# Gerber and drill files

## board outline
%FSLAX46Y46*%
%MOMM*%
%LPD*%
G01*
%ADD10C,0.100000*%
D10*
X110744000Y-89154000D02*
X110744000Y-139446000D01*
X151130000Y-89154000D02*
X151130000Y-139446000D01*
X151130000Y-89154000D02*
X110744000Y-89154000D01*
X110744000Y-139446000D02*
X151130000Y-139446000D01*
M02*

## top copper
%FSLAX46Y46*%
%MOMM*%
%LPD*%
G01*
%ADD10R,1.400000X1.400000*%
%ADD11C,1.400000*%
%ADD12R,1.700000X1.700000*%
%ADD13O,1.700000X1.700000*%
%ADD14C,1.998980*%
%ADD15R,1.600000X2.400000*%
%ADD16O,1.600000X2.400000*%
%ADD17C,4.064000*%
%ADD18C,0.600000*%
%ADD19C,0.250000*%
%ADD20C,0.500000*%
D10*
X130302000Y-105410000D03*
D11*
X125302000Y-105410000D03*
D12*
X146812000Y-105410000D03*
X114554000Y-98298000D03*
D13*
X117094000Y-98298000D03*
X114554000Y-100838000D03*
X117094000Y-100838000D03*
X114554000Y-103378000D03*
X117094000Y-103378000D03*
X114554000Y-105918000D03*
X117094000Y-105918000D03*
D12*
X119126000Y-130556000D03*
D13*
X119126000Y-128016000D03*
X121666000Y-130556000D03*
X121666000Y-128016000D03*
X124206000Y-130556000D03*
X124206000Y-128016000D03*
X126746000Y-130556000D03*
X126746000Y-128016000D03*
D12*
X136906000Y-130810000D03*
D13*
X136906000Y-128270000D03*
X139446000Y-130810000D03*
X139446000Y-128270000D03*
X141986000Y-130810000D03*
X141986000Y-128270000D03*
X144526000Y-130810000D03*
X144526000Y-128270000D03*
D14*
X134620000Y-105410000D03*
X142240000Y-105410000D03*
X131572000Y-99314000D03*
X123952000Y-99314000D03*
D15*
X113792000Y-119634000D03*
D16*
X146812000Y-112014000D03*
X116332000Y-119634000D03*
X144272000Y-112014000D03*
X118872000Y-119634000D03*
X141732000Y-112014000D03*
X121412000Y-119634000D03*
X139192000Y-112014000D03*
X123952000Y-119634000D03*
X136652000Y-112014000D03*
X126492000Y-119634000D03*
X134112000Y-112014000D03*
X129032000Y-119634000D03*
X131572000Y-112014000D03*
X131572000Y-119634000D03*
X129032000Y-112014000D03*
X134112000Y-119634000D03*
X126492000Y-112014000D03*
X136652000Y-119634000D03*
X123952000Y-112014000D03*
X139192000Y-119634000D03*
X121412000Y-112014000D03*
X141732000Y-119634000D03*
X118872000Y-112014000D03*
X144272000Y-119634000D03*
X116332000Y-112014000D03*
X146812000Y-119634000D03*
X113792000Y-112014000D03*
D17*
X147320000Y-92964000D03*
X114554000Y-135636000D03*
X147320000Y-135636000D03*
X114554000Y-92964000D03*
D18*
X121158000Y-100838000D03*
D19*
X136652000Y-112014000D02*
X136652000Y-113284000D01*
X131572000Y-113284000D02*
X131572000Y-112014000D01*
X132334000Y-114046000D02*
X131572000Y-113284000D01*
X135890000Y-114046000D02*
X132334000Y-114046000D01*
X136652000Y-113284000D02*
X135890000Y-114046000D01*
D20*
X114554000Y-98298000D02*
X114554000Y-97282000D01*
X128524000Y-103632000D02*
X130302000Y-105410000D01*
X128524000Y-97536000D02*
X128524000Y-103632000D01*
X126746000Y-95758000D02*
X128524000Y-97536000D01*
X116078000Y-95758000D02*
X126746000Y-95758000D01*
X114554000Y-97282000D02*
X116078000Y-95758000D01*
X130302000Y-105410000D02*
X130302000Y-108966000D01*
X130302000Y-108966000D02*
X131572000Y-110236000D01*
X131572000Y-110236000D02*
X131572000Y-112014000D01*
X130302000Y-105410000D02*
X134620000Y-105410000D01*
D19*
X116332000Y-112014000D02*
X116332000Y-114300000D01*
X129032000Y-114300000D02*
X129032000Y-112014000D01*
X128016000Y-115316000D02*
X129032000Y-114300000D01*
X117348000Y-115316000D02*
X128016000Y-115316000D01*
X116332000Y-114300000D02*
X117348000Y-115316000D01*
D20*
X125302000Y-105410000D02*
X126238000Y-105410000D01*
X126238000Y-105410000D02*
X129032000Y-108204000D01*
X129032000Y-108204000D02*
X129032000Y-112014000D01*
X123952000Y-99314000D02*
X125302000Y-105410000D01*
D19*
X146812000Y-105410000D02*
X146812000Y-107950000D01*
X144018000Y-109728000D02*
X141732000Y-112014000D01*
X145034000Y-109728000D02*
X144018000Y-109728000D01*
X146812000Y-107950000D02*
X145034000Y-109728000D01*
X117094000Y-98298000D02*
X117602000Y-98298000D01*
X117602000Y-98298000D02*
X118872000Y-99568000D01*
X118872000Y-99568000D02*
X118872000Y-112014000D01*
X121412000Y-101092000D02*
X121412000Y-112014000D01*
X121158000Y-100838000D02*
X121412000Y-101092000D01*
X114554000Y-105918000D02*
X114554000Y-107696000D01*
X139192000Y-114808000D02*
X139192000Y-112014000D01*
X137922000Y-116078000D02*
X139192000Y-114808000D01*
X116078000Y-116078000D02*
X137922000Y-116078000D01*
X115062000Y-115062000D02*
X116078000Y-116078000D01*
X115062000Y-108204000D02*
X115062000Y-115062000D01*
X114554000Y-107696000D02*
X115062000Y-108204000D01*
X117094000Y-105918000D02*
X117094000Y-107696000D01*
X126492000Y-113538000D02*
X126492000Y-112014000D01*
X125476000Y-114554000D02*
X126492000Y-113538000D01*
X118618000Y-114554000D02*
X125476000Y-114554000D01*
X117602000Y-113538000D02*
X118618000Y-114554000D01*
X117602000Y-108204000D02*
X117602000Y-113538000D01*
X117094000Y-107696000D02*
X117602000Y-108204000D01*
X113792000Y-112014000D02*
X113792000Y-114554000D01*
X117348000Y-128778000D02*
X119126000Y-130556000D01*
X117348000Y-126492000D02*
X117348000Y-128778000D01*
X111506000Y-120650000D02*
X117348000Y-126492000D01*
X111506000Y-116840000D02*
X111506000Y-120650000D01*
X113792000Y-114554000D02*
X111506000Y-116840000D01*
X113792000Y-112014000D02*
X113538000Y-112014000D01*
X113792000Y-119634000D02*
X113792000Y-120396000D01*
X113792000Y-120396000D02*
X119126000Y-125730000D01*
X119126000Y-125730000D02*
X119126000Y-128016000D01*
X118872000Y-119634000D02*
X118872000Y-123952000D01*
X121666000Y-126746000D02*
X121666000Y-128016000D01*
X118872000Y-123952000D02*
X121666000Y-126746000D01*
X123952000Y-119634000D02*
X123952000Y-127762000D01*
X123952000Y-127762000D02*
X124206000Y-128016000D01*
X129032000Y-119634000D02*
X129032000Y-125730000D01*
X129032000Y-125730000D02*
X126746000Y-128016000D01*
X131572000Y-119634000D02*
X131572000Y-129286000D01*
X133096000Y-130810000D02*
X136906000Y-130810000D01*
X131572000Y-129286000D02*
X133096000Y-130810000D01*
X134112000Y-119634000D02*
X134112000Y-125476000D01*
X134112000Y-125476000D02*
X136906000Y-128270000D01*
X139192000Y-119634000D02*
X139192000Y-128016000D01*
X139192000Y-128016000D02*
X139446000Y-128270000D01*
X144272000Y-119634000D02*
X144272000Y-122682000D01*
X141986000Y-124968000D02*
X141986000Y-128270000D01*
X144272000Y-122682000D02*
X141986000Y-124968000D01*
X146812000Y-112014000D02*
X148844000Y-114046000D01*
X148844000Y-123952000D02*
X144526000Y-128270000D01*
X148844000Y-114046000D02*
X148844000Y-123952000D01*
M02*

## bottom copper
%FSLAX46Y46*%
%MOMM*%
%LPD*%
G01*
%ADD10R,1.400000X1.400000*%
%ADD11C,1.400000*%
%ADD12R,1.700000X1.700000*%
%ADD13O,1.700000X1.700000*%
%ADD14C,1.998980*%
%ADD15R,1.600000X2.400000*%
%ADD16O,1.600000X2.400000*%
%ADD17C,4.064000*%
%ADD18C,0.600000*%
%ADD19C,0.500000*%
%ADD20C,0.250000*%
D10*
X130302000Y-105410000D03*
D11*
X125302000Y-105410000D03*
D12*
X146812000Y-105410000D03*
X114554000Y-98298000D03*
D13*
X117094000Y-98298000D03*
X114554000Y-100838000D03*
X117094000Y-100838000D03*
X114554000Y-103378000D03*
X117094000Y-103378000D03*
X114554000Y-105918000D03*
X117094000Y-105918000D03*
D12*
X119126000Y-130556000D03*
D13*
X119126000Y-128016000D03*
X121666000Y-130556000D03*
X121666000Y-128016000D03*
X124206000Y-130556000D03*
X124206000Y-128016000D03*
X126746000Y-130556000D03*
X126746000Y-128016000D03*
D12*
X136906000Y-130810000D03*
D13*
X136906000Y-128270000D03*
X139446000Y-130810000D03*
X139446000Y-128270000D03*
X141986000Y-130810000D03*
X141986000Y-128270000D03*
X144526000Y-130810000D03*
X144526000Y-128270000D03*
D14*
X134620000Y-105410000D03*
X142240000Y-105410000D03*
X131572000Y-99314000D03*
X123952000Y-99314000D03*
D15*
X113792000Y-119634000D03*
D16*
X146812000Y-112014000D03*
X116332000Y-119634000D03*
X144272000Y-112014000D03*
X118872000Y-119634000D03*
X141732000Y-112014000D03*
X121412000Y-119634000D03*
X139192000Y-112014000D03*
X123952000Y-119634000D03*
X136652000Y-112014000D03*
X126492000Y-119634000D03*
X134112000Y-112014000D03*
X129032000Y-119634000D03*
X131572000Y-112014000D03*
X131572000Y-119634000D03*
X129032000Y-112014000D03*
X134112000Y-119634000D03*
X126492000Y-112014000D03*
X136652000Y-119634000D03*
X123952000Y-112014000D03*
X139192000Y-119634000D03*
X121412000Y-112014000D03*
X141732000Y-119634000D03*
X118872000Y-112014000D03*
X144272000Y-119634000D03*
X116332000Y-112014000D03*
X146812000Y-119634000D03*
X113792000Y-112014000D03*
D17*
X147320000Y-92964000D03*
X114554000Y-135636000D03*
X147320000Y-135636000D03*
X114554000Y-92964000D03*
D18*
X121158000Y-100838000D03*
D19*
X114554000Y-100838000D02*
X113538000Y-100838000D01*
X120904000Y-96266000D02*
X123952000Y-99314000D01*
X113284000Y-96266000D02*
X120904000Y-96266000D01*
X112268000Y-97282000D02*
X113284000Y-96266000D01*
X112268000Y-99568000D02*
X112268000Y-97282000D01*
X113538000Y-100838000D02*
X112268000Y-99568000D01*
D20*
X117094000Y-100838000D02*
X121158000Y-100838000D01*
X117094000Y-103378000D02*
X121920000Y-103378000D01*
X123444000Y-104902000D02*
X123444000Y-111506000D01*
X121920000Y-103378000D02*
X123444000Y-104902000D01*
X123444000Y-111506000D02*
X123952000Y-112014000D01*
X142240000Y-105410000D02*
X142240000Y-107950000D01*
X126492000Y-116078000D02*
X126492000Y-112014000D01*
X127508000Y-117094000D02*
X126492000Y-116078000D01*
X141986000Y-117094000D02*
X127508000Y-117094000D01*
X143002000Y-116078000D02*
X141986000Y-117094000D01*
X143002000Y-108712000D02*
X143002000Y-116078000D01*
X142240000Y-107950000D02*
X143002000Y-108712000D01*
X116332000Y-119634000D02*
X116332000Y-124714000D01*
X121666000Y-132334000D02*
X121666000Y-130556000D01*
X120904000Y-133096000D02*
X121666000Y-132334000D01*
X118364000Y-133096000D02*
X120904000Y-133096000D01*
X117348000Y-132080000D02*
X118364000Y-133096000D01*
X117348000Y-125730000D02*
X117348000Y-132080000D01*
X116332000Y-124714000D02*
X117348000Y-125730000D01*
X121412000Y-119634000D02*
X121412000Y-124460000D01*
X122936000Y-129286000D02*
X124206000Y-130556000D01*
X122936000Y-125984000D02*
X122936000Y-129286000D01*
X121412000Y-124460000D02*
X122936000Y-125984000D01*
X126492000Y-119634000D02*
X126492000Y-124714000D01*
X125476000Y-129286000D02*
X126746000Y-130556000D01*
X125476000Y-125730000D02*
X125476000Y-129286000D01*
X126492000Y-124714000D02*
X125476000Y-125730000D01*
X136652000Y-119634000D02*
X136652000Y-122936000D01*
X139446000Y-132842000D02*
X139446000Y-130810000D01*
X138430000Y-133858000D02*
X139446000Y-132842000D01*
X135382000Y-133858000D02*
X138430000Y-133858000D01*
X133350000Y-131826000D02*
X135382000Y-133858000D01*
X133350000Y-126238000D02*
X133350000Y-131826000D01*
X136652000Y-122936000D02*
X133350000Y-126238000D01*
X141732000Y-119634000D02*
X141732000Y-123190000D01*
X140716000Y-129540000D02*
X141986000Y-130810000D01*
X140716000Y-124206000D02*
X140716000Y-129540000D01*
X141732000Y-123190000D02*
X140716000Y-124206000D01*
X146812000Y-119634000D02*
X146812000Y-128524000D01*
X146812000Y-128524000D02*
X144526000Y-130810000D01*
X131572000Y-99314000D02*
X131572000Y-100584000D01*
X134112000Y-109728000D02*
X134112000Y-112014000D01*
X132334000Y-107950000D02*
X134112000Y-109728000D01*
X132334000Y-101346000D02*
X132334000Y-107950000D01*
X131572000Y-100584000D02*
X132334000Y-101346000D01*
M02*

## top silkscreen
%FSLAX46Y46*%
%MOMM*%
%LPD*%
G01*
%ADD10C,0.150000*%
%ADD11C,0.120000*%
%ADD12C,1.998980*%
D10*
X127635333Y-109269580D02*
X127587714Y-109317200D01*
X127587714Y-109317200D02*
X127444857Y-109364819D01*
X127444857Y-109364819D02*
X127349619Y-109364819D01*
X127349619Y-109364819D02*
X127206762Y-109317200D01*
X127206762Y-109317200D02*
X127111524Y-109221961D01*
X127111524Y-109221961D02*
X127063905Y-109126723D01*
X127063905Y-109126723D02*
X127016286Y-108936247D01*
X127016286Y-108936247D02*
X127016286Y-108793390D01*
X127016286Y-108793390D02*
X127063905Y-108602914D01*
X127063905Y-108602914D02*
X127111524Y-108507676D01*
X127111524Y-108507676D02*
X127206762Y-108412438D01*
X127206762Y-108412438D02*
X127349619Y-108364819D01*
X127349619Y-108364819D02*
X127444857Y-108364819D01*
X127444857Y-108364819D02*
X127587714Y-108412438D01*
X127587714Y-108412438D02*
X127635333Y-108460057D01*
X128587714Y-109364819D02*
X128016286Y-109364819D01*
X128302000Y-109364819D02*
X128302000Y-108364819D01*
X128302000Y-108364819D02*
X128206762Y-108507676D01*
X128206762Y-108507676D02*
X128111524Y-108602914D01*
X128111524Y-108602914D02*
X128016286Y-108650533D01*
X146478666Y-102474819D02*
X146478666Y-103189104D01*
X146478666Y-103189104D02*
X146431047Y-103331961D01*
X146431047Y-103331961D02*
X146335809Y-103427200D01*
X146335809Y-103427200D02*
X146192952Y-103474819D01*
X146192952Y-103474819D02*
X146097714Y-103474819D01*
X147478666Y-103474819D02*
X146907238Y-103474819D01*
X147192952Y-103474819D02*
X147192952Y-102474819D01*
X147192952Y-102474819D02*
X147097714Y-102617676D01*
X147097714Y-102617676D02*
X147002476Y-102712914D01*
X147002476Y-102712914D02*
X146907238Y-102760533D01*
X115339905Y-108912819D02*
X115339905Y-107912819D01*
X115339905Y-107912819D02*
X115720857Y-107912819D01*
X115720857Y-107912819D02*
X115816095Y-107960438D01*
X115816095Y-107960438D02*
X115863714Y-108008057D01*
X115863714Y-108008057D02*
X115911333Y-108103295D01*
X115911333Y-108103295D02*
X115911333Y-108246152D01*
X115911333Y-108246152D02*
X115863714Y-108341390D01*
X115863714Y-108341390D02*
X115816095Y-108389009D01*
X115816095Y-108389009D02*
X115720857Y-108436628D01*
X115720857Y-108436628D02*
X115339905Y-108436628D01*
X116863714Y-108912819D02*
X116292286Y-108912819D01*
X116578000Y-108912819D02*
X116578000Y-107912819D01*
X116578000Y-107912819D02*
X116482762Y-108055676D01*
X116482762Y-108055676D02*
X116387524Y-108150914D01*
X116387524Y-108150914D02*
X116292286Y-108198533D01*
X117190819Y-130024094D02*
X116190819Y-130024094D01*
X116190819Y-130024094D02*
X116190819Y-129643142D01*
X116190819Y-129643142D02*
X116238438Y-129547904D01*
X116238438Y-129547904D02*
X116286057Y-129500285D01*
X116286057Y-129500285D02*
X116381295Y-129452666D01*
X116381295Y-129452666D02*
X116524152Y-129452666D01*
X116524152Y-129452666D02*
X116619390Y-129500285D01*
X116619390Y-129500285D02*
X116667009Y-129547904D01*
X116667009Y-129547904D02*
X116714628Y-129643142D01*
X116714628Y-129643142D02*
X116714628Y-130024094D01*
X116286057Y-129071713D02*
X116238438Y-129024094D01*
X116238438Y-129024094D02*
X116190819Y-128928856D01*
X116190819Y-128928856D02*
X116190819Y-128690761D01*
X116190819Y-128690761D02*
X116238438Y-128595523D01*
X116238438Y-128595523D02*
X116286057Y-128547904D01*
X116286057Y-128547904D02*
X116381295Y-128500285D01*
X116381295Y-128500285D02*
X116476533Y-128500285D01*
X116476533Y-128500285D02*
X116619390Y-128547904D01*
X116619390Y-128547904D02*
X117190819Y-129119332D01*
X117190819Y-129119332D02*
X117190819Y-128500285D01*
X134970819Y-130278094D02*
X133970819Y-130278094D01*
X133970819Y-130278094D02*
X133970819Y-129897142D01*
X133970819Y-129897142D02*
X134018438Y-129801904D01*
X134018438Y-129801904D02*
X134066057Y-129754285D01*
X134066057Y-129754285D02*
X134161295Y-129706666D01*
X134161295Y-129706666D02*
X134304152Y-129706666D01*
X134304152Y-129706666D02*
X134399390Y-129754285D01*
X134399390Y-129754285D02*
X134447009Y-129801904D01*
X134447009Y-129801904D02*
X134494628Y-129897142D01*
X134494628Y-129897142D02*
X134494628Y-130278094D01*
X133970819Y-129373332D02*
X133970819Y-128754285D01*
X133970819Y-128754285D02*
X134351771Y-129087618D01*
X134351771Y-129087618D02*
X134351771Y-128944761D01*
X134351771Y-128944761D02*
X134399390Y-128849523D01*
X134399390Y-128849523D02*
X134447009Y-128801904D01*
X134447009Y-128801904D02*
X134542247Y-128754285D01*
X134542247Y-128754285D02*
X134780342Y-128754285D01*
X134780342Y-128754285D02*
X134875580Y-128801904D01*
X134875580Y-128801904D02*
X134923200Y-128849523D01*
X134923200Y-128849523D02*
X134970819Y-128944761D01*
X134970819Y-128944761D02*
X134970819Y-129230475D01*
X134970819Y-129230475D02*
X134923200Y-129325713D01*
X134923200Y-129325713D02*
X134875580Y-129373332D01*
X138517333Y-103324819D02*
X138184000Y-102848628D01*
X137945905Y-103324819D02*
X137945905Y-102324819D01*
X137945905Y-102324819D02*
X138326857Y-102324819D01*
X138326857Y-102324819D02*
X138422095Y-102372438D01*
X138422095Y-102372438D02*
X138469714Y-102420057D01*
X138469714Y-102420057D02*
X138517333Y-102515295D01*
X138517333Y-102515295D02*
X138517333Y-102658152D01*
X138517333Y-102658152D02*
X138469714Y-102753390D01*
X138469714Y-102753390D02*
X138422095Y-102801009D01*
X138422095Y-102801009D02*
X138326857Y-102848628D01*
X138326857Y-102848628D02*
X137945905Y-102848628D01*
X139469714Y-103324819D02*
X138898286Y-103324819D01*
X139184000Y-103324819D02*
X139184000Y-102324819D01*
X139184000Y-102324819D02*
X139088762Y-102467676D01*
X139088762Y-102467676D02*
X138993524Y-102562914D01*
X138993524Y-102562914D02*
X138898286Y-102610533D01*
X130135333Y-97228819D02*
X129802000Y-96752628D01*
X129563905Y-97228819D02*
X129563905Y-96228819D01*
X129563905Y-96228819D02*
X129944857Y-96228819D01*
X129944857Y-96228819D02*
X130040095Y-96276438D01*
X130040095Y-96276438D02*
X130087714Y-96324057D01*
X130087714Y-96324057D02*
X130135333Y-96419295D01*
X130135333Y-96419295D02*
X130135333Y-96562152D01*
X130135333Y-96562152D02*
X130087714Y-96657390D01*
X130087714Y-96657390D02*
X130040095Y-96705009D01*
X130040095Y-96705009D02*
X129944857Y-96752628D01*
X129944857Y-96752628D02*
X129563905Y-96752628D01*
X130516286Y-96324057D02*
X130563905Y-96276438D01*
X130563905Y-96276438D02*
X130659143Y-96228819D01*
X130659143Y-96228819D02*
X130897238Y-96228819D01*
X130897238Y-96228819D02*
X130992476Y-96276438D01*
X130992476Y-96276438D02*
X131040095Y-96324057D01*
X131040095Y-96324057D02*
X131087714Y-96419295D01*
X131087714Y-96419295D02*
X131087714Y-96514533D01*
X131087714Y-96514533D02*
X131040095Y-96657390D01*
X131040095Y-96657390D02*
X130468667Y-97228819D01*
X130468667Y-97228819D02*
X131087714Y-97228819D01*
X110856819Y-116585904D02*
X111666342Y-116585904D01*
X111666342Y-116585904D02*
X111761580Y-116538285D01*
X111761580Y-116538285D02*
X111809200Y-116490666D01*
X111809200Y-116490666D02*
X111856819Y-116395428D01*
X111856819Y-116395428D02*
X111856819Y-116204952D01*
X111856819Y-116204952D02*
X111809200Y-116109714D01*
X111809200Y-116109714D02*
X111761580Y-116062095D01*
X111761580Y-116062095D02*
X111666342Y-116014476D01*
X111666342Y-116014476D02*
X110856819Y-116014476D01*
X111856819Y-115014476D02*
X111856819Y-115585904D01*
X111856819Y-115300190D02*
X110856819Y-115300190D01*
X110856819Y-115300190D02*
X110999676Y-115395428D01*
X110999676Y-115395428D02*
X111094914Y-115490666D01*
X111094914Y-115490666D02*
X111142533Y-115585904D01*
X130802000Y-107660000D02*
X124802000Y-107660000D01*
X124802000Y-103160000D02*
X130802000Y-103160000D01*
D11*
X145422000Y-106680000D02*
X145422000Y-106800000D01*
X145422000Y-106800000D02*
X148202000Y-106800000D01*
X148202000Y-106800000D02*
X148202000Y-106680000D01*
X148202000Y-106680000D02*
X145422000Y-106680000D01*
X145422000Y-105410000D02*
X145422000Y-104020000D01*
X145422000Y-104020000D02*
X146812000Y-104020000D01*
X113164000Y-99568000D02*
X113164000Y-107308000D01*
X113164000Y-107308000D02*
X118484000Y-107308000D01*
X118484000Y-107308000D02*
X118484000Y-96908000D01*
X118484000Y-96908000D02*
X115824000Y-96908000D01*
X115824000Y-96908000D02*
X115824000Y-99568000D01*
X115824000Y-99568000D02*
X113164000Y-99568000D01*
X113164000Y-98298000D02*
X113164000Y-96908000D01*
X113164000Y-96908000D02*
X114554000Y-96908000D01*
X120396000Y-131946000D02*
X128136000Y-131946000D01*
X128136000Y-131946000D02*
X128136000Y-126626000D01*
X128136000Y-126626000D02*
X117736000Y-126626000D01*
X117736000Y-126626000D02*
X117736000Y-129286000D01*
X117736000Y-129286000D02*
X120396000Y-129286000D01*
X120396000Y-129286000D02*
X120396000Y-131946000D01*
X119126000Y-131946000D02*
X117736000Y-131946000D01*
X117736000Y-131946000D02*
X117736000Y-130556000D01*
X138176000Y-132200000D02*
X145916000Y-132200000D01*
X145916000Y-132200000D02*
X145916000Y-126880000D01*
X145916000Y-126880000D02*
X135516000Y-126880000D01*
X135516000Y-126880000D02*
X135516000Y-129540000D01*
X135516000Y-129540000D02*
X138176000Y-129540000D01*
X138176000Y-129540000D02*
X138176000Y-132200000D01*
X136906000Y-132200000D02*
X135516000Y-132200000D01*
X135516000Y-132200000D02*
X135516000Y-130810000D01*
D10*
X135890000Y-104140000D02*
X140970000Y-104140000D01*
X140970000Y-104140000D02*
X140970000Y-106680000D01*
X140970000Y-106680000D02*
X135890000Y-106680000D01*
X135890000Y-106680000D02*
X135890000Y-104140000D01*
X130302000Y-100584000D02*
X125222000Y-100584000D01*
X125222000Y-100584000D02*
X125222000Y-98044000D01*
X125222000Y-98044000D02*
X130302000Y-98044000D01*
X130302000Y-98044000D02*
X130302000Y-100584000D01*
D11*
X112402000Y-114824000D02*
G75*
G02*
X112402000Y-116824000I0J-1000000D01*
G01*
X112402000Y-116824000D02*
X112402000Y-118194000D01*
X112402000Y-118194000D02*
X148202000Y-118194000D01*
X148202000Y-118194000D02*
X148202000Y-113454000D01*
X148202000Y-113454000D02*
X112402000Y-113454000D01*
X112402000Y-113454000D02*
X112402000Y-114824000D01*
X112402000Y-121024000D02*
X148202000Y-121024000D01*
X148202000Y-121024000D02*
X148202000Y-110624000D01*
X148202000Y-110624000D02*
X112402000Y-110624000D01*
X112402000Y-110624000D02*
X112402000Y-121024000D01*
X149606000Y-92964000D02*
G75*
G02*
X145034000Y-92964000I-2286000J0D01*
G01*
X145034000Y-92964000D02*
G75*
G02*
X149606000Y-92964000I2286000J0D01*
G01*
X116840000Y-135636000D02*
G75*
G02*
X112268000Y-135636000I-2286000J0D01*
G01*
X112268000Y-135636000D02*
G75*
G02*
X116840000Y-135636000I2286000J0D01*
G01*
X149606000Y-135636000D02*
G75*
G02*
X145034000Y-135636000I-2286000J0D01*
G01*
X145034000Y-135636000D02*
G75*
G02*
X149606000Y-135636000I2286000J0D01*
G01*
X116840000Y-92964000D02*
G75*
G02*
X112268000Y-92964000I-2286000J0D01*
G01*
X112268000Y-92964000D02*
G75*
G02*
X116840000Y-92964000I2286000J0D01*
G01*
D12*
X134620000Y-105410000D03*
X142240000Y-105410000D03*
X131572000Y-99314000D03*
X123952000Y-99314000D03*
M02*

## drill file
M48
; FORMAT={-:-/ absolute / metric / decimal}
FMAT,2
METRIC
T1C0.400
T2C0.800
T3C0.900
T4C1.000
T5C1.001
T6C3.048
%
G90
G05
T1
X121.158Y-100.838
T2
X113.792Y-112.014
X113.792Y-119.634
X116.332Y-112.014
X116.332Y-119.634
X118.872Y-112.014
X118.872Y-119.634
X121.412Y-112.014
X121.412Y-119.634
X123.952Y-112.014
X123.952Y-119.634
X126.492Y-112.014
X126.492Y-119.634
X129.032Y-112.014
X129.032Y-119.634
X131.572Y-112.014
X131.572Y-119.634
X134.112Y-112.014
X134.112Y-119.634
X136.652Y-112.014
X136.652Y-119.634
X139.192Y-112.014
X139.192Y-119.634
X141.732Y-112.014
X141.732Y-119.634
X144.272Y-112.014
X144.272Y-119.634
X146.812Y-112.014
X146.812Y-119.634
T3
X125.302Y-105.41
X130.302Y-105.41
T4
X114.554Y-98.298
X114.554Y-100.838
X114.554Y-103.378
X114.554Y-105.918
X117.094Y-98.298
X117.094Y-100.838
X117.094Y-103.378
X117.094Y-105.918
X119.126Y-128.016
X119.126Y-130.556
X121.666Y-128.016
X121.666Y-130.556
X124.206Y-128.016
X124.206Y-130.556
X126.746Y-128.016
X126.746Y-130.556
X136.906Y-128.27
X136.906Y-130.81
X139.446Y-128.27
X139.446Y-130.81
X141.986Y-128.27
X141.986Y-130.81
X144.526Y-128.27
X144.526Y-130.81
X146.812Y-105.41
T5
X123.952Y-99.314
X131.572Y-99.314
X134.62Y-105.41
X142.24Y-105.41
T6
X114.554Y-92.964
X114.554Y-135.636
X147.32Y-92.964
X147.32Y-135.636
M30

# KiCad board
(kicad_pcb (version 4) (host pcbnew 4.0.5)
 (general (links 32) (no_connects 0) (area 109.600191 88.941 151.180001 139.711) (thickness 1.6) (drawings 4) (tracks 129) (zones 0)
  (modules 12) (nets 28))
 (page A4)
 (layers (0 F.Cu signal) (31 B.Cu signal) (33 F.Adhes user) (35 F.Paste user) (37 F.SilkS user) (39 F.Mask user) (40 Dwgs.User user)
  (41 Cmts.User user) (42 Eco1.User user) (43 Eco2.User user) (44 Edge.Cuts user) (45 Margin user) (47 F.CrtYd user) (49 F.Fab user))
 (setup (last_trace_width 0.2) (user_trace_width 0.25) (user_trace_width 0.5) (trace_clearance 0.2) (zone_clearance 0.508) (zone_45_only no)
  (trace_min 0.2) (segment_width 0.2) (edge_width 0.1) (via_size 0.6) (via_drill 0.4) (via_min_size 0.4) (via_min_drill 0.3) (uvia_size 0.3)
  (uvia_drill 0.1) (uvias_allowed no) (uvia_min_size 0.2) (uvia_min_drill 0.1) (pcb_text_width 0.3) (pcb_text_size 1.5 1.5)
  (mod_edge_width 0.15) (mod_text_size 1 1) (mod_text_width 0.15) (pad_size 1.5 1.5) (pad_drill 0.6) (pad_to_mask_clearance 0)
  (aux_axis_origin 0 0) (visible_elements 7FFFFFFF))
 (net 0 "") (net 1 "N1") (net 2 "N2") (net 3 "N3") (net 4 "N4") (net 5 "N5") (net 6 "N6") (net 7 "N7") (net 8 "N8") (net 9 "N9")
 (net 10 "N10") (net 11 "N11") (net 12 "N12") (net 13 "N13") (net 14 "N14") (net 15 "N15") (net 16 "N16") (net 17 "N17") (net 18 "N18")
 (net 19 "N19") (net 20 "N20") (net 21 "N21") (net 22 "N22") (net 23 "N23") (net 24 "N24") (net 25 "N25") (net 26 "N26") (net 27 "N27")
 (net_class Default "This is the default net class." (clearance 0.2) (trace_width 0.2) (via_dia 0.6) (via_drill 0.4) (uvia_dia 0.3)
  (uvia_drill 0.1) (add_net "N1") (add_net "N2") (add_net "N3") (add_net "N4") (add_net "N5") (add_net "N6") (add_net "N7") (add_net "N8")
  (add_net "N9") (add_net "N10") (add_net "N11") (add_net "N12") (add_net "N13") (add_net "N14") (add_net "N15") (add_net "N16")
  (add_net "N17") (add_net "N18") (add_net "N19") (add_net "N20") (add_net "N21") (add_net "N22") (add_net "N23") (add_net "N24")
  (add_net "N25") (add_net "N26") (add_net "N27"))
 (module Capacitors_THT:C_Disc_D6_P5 (layer F.Cu) (at 130.302 105.41 180)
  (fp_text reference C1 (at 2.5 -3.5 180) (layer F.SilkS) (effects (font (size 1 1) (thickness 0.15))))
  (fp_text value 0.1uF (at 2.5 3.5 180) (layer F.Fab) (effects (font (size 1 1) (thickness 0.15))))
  (fp_line (start -0.5 -2.25) (end 5.5 -2.25) (layer F.SilkS) (width 0.15))
  (fp_line (start 5.5 2.25) (end -0.5 2.25) (layer F.SilkS) (width 0.15))
  (pad 1 thru_hole rect (at 0 0 180) (size 1.4 1.4) (drill 0.9) (layers *.Cu *.Mask) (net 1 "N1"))
  (pad 2 thru_hole circle (at 5 0 180) (size 1.4 1.4) (drill 0.9) (layers *.Cu *.Mask) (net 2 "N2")))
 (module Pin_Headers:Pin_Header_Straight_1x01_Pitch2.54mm (layer F.Cu) (at 146.812 105.41)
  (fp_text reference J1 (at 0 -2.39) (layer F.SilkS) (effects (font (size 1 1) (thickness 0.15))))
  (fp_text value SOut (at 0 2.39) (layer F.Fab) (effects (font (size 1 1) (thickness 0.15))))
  (fp_line (start -1.39 1.27) (end -1.39 1.39) (layer F.SilkS) (width 0.12))
  (fp_line (start -1.39 1.39) (end 1.39 1.39) (layer F.SilkS) (width 0.12))
  (fp_line (start 1.39 1.39) (end 1.39 1.27) (layer F.SilkS) (width 0.12))
  (fp_line (start 1.39 1.27) (end -1.39 1.27) (layer F.SilkS) (width 0.12))
  (fp_line (start -1.39 0) (end -1.39 -1.39) (layer F.SilkS) (width 0.12))
  (fp_line (start -1.39 -1.39) (end 0 -1.39) (layer F.SilkS) (width 0.12))
  (pad 1 thru_hole rect (at 0 0) (size 1.7 1.7) (drill 1) (layers *.Cu *.Mask) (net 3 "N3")))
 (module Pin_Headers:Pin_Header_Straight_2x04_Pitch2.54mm (layer F.Cu) (at 114.554 98.298)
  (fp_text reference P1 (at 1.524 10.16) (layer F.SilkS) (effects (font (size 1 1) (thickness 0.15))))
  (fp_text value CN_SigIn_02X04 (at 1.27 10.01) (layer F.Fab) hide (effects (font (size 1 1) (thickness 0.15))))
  (fp_line (start -1.39 1.27) (end -1.39 9.01) (layer F.SilkS) (width 0.12))
  (fp_line (start -1.39 9.01) (end 3.93 9.01) (layer F.SilkS) (width 0.12))
  (fp_line (start 3.93 9.01) (end 3.93 -1.39) (layer F.SilkS) (width 0.12))
  (fp_line (start 3.93 -1.39) (end 1.27 -1.39) (layer F.SilkS) (width 0.12))
  (fp_line (start 1.27 -1.39) (end 1.27 1.27) (layer F.SilkS) (width 0.12))
  (fp_line (start 1.27 1.27) (end -1.39 1.27) (layer F.SilkS) (width 0.12))
  (fp_line (start -1.39 0) (end -1.39 -1.39) (layer F.SilkS) (width 0.12))
  (fp_line (start -1.39 -1.39) (end 0 -1.39) (layer F.SilkS) (width 0.12))
  (pad 1 thru_hole rect (at 0 0) (size 1.7 1.7) (drill 1) (layers *.Cu *.Mask) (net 1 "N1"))
  (pad 2 thru_hole oval (at 2.54 0) (size 1.7 1.7) (drill 1) (layers *.Cu *.Mask) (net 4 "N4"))
  (pad 3 thru_hole oval (at 0 2.54) (size 1.7 1.7) (drill 1) (layers *.Cu *.Mask) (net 2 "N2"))
  (pad 4 thru_hole oval (at 2.54 2.54) (size 1.7 1.7) (drill 1) (layers *.Cu *.Mask) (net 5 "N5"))
  (pad 5 thru_hole oval (at 0 5.08) (size 1.7 1.7) (drill 1) (layers *.Cu *.Mask) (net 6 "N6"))
  (pad 6 thru_hole oval (at 2.54 5.08) (size 1.7 1.7) (drill 1) (layers *.Cu *.Mask) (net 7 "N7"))
  (pad 7 thru_hole oval (at 0 7.62) (size 1.7 1.7) (drill 1) (layers *.Cu *.Mask) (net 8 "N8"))
  (pad 8 thru_hole oval (at 2.54 7.62) (size 1.7 1.7) (drill 1) (layers *.Cu *.Mask) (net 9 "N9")))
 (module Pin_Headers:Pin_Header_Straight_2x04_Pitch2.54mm (layer F.Cu) (at 119.126 130.556 90)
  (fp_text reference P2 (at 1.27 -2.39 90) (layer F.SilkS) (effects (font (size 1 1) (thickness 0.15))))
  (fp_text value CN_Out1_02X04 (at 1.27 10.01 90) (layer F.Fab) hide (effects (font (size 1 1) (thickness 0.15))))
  (fp_line (start -1.39 1.27) (end -1.39 9.01) (layer F.SilkS) (width 0.12))
  (fp_line (start -1.39 9.01) (end 3.93 9.01) (layer F.SilkS) (width 0.12))
  (fp_line (start 3.93 9.01) (end 3.93 -1.39) (layer F.SilkS) (width 0.12))
  (fp_line (start 3.93 -1.39) (end 1.27 -1.39) (layer F.SilkS) (width 0.12))
  (fp_line (start 1.27 -1.39) (end 1.27 1.27) (layer F.SilkS) (width 0.12))
  (fp_line (start 1.27 1.27) (end -1.39 1.27) (layer F.SilkS) (width 0.12))
  (fp_line (start -1.39 0) (end -1.39 -1.39) (layer F.SilkS) (width 0.12))
  (fp_line (start -1.39 -1.39) (end 0 -1.39) (layer F.SilkS) (width 0.12))
  (pad 1 thru_hole rect (at 0 0 90) (size 1.7 1.7) (drill 1) (layers *.Cu *.Mask) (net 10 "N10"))
  (pad 2 thru_hole oval (at 2.54 0 90) (size 1.7 1.7) (drill 1) (layers *.Cu *.Mask) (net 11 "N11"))
  (pad 3 thru_hole oval (at 0 2.54 90) (size 1.7 1.7) (drill 1) (layers *.Cu *.Mask) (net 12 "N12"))
  (pad 4 thru_hole oval (at 2.54 2.54 90) (size 1.7 1.7) (drill 1) (layers *.Cu *.Mask) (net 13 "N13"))
  (pad 5 thru_hole oval (at 0 5.08 90) (size 1.7 1.7) (drill 1) (layers *.Cu *.Mask) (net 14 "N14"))
  (pad 6 thru_hole oval (at 2.54 5.08 90) (size 1.7 1.7) (drill 1) (layers *.Cu *.Mask) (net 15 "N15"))
  (pad 7 thru_hole oval (at 0 7.62 90) (size 1.7 1.7) (drill 1) (layers *.Cu *.Mask) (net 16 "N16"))
  (pad 8 thru_hole oval (at 2.54 7.62 90) (size 1.7 1.7) (drill 1) (layers *.Cu *.Mask) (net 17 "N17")))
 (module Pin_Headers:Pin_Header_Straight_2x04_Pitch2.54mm (layer F.Cu) (at 136.906 130.81 90)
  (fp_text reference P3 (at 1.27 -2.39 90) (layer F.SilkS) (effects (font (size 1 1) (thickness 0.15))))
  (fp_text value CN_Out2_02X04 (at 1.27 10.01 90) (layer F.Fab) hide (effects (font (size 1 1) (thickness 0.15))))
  (fp_line (start -1.39 1.27) (end -1.39 9.01) (layer F.SilkS) (width 0.12))
  (fp_line (start -1.39 9.01) (end 3.93 9.01) (layer F.SilkS) (width 0.12))
  (fp_line (start 3.93 9.01) (end 3.93 -1.39) (layer F.SilkS) (width 0.12))
  (fp_line (start 3.93 -1.39) (end 1.27 -1.39) (layer F.SilkS) (width 0.12))
  (fp_line (start 1.27 -1.39) (end 1.27 1.27) (layer F.SilkS) (width 0.12))
  (fp_line (start 1.27 1.27) (end -1.39 1.27) (layer F.SilkS) (width 0.12))
  (fp_line (start -1.39 0) (end -1.39 -1.39) (layer F.SilkS) (width 0.12))
  (fp_line (start -1.39 -1.39) (end 0 -1.39) (layer F.SilkS) (width 0.12))
  (pad 1 thru_hole rect (at 0 0 90) (size 1.7 1.7) (drill 1) (layers *.Cu *.Mask) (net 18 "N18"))
  (pad 2 thru_hole oval (at 2.54 0 90) (size 1.7 1.7) (drill 1) (layers *.Cu *.Mask) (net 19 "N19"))
  (pad 3 thru_hole oval (at 0 2.54 90) (size 1.7 1.7) (drill 1) (layers *.Cu *.Mask) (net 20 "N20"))
  (pad 4 thru_hole oval (at 2.54 2.54 90) (size 1.7 1.7) (drill 1) (layers *.Cu *.Mask) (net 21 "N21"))
  (pad 5 thru_hole oval (at 0 5.08 90) (size 1.7 1.7) (drill 1) (layers *.Cu *.Mask) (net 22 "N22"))
  (pad 6 thru_hole oval (at 2.54 5.08 90) (size 1.7 1.7) (drill 1) (layers *.Cu *.Mask) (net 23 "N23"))
  (pad 7 thru_hole oval (at 0 7.62 90) (size 1.7 1.7) (drill 1) (layers *.Cu *.Mask) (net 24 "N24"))
  (pad 8 thru_hole oval (at 2.54 7.62 90) (size 1.7 1.7) (drill 1) (layers *.Cu *.Mask) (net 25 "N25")))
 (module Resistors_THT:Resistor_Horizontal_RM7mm (layer F.Cu) (at 134.62 105.41)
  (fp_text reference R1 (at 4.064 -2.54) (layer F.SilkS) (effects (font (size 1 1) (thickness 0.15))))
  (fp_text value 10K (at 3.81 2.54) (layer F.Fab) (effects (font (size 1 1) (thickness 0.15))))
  (fp_line (start 1.27 -1.27) (end 6.35 -1.27) (layer F.SilkS) (width 0.15))
  (fp_line (start 6.35 -1.27) (end 6.35 1.27) (layer F.SilkS) (width 0.15))
  (fp_line (start 6.35 1.27) (end 1.27 1.27) (layer F.SilkS) (width 0.15))
  (fp_line (start 1.27 1.27) (end 1.27 -1.27) (layer F.SilkS) (width 0.15))
  (pad 1 thru_hole circle (at 0 0) (size 1.99898 1.99898) (drill 1.00076) (layers *.Cu *.SilkS *.Mask) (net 1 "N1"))
  (pad 2 thru_hole circle (at 7.62 0) (size 1.99898 1.99898) (drill 1.00076) (layers *.Cu *.SilkS *.Mask) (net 9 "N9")))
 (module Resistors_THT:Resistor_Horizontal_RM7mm (layer F.Cu) (at 131.572 99.314 180)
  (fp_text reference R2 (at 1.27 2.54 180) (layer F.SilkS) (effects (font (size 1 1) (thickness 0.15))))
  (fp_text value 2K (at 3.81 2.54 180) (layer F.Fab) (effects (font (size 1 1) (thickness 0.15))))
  (fp_line (start 1.27 -1.27) (end 6.35 -1.27) (layer F.SilkS) (width 0.15))
  (fp_line (start 6.35 -1.27) (end 6.35 1.27) (layer F.SilkS) (width 0.15))
  (fp_line (start 6.35 1.27) (end 1.27 1.27) (layer F.SilkS) (width 0.15))
  (fp_line (start 1.27 1.27) (end 1.27 -1.27) (layer F.SilkS) (width 0.15))
  (pad 1 thru_hole circle (at 0 0 180) (size 1.99898 1.99898) (drill 1.00076) (layers *.Cu *.SilkS *.Mask) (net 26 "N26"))
  (pad 2 thru_hole circle (at 7.62 0 180) (size 1.99898 1.99898) (drill 1.00076) (layers *.Cu *.SilkS *.Mask) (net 2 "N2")))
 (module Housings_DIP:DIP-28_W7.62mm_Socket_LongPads (layer F.Cu) (at 113.792 119.634 90)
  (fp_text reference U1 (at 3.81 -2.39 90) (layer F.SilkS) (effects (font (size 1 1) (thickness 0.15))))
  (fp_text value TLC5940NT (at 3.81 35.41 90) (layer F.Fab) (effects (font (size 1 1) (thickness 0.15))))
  (fp_arc (start 3.81 -1.39) (end 2.81 -1.39) (angle -180) (layer F.SilkS) (width 0.12))
  (fp_line (start 2.81 -1.39) (end 1.44 -1.39) (layer F.SilkS) (width 0.12))
  (fp_line (start 1.44 -1.39) (end 1.44 34.41) (layer F.SilkS) (width 0.12))
  (fp_line (start 1.44 34.41) (end 6.18 34.41) (layer F.SilkS) (width 0.12))
  (fp_line (start 6.18 34.41) (end 6.18 -1.39) (layer F.SilkS) (width 0.12))
  (fp_line (start 6.18 -1.39) (end 4.81 -1.39) (layer F.SilkS) (width 0.12))
  (fp_line (start -1.39 -1.39) (end -1.39 34.41) (layer F.SilkS) (width 0.12))
  (fp_line (start -1.39 34.41) (end 9.01 34.41) (layer F.SilkS) (width 0.12))
  (fp_line (start 9.01 34.41) (end 9.01 -1.39) (layer F.SilkS) (width 0.12))
  (fp_line (start 9.01 -1.39) (end -1.39 -1.39) (layer F.SilkS) (width 0.12))
  (pad 1 thru_hole rect (at 0 0 90) (size 2.4 1.6) (drill 0.8) (layers *.Cu *.Mask) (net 11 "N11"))
  (pad 15 thru_hole oval (at 7.62 33.02 90) (size 2.4 1.6) (drill 0.8) (layers *.Cu *.Mask) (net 25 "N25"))
  (pad 2 thru_hole oval (at 0 2.54 90) (size 2.4 1.6) (drill 0.8) (layers *.Cu *.Mask) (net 12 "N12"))
  (pad 16 thru_hole oval (at 7.62 30.48 90) (size 2.4 1.6) (drill 0.8) (layers *.Cu *.Mask) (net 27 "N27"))
  (pad 3 thru_hole oval (at 0 5.08 90) (size 2.4 1.6) (drill 0.8) (layers *.Cu *.Mask) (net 13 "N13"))
  (pad 17 thru_hole oval (at 7.62 27.94 90) (size 2.4 1.6) (drill 0.8) (layers *.Cu *.Mask) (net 3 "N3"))
  (pad 4 thru_hole oval (at 0 7.62 90) (size 2.4 1.6) (drill 0.8) (layers *.Cu *.Mask) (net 14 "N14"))
  (pad 18 thru_hole oval (at 7.62 25.4 90) (size 2.4 1.6) (drill 0.8) (layers *.Cu *.Mask) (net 8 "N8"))
  (pad 5 thru_hole oval (at 0 10.16 90) (size 2.4 1.6) (drill 0.8) (layers *.Cu *.Mask) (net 15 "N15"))
  (pad 19 thru_hole oval (at 7.62 22.86 90) (size 2.4 1.6) (drill 0.8) (layers *.Cu *.Mask) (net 1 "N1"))
  (pad 6 thru_hole oval (at 0 12.7 90) (size 2.4 1.6) (drill 0.8) (layers *.Cu *.Mask) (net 16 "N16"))
  (pad 20 thru_hole oval (at 7.62 20.32 90) (size 2.4 1.6) (drill 0.8) (layers *.Cu *.Mask) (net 26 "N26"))
  (pad 7 thru_hole oval (at 0 15.24 90) (size 2.4 1.6) (drill 0.8) (layers *.Cu *.Mask) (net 17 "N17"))
  (pad 21 thru_hole oval (at 7.62 17.78 90) (size 2.4 1.6) (drill 0.8) (layers *.Cu *.Mask) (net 1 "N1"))
  (pad 8 thru_hole oval (at 0 17.78 90) (size 2.4 1.6) (drill 0.8) (layers *.Cu *.Mask) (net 18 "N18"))
  (pad 22 thru_hole oval (at 7.62 15.24 90) (size 2.4 1.6) (drill 0.8) (layers *.Cu *.Mask) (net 2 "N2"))
  (pad 9 thru_hole oval (at 0 20.32 90) (size 2.4 1.6) (drill 0.8) (layers *.Cu *.Mask) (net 19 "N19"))
  (pad 23 thru_hole oval (at 7.62 12.7 90) (size 2.4 1.6) (drill 0.8) (layers *.Cu *.Mask) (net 9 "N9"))
  (pad 10 thru_hole oval (at 0 22.86 90) (size 2.4 1.6) (drill 0.8) (layers *.Cu *.Mask) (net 20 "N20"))
  (pad 24 thru_hole oval (at 7.62 10.16 90) (size 2.4 1.6) (drill 0.8) (layers *.Cu *.Mask) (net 7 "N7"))
  (pad 11 thru_hole oval (at 0 25.4 90) (size 2.4 1.6) (drill 0.8) (layers *.Cu *.Mask) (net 21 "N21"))
  (pad 25 thru_hole oval (at 7.62 7.62 90) (size 2.4 1.6) (drill 0.8) (layers *.Cu *.Mask) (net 5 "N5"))
  (pad 12 thru_hole oval (at 0 27.94 90) (size 2.4 1.6) (drill 0.8) (layers *.Cu *.Mask) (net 22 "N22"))
  (pad 26 thru_hole oval (at 7.62 5.08 90) (size 2.4 1.6) (drill 0.8) (layers *.Cu *.Mask) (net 4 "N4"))
  (pad 13 thru_hole oval (at 0 30.48 90) (size 2.4 1.6) (drill 0.8) (layers *.Cu *.Mask) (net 23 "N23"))
  (pad 27 thru_hole oval (at 7.62 2.54 90) (size 2.4 1.6) (drill 0.8) (layers *.Cu *.Mask) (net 2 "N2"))
  (pad 14 thru_hole oval (at 0 33.02 90) (size 2.4 1.6) (drill 0.8) (layers *.Cu *.Mask) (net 24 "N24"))
  (pad 28 thru_hole oval (at 7.62 0 90) (size 2.4 1.6) (drill 0.8) (layers *.Cu *.Mask) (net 10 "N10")))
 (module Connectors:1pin (layer F.Cu) (at 147.32 92.964)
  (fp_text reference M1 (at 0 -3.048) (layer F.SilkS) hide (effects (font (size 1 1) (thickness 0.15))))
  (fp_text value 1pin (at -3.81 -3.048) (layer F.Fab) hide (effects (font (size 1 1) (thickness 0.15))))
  (fp_circle (center 0 0) (end 0 -2.286) (layer F.SilkS) (width 0.12))
  (pad 1 thru_hole circle (at 0 0) (size 4.064 4.064) (drill 3.048) (layers *.Cu *.Mask)))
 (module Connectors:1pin (layer F.Cu) (at 114.554 135.636)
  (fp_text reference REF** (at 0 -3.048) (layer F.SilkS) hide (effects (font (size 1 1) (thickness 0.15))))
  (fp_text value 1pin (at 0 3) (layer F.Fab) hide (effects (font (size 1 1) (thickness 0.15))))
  (fp_circle (center 0 0) (end 0 -2.286) (layer F.SilkS) (width 0.12))
  (pad 1 thru_hole circle (at 0 0) (size 4.064 4.064) (drill 3.048) (layers *.Cu *.Mask)))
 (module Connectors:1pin (layer F.Cu) (at 147.32 135.636)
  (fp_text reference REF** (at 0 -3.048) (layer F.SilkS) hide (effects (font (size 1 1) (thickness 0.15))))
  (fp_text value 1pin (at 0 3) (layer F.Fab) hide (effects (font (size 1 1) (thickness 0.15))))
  (fp_circle (center 0 0) (end 0 -2.286) (layer F.SilkS) (width 0.12))
  (pad 1 thru_hole circle (at 0 0) (size 4.064 4.064) (drill 3.048) (layers *.Cu *.Mask)))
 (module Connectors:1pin (layer F.Cu) (at 114.554 92.964)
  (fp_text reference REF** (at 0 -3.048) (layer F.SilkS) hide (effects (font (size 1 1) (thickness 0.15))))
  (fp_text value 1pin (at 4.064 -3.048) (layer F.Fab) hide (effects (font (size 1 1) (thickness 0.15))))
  (fp_circle (center 0 0) (end 0 -2.286) (layer F.SilkS) (width 0.12))
  (pad 1 thru_hole circle (at 0 0) (size 4.064 4.064) (drill 3.048) (layers *.Cu *.Mask)))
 (gr_line (start 110.744 89.154) (end 110.744 139.446) (angle 90) (layer Edge.Cuts) (width 0.1))
 (gr_line (start 151.13 89.154) (end 151.13 139.446) (angle 90) (layer Edge.Cuts) (width 0.1))
 (gr_line (start 151.13 89.154) (end 110.744 89.154) (angle 90) (layer Edge.Cuts) (width 0.1))
 (gr_line (start 110.744 139.446) (end 151.13 139.446) (angle 90) (layer Edge.Cuts) (width 0.1))
 (segment (start 136.652 112.014) (end 136.652 113.284) (width 0.25) (layer F.Cu) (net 1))
 (segment (start 131.572 113.284) (end 131.572 112.014) (width 0.25) (layer F.Cu) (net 1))
 (segment (start 132.334 114.046) (end 131.572 113.284) (width 0.25) (layer F.Cu) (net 1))
 (segment (start 135.89 114.046) (end 132.334 114.046) (width 0.25) (layer F.Cu) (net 1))
 (segment (start 136.652 113.284) (end 135.89 114.046) (width 0.25) (layer F.Cu) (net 1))
 (segment (start 114.554 98.298) (end 114.554 97.282) (width 0.5) (layer F.Cu) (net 1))
 (segment (start 128.524 103.632) (end 130.302 105.41) (width 0.5) (layer F.Cu) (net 1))
 (segment (start 128.524 97.536) (end 128.524 103.632) (width 0.5) (layer F.Cu) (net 1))
 (segment (start 126.746 95.758) (end 128.524 97.536) (width 0.5) (layer F.Cu) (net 1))
 (segment (start 116.078 95.758) (end 126.746 95.758) (width 0.5) (layer F.Cu) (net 1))
 (segment (start 114.554 97.282) (end 116.078 95.758) (width 0.5) (layer F.Cu) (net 1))
 (segment (start 130.302 105.41) (end 130.302 108.966) (width 0.5) (layer F.Cu) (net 1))
 (segment (start 130.302 108.966) (end 131.572 110.236) (width 0.5) (layer F.Cu) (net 1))
 (segment (start 131.572 110.236) (end 131.572 112.014) (width 0.5) (layer F.Cu) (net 1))
 (segment (start 130.302 105.41) (end 134.62 105.41) (width 0.5) (layer F.Cu) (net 1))
 (segment (start 114.554 100.838) (end 113.538 100.838) (width 0.5) (layer B.Cu) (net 2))
 (segment (start 120.904 96.266) (end 123.952 99.314) (width 0.5) (layer B.Cu) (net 2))
 (segment (start 113.284 96.266) (end 120.904 96.266) (width 0.5) (layer B.Cu) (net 2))
 (segment (start 112.268 97.282) (end 113.284 96.266) (width 0.5) (layer B.Cu) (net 2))
 (segment (start 112.268 99.568) (end 112.268 97.282) (width 0.5) (layer B.Cu) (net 2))
 (segment (start 113.538 100.838) (end 112.268 99.568) (width 0.5) (layer B.Cu) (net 2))
 (segment (start 116.332 112.014) (end 116.332 114.3) (width 0.25) (layer F.Cu) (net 2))
 (segment (start 129.032 114.3) (end 129.032 112.014) (width 0.25) (layer F.Cu) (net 2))
 (segment (start 128.016 115.316) (end 129.032 114.3) (width 0.25) (layer F.Cu) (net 2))
 (segment (start 117.348 115.316) (end 128.016 115.316) (width 0.25) (layer F.Cu) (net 2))
 (segment (start 116.332 114.3) (end 117.348 115.316) (width 0.25) (layer F.Cu) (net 2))
 (segment (start 125.302 105.41) (end 126.238 105.41) (width 0.5) (layer F.Cu) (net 2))
 (segment (start 126.238 105.41) (end 129.032 108.204) (width 0.5) (layer F.Cu) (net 2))
 (segment (start 129.032 108.204) (end 129.032 112.014) (width 0.5) (layer F.Cu) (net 2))
 (segment (start 123.952 99.314) (end 125.302 105.41) (width 0.5) (layer F.Cu) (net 2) (status 10))
 (segment (start 146.812 105.41) (end 146.812 107.95) (width 0.25) (layer F.Cu) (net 3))
 (segment (start 144.018 109.728) (end 141.732 112.014) (width 0.25) (layer F.Cu) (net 3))
 (segment (start 145.034 109.728) (end 144.018 109.728) (width 0.25) (layer F.Cu) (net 3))
 (segment (start 146.812 107.95) (end 145.034 109.728) (width 0.25) (layer F.Cu) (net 3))
 (segment (start 117.094 98.298) (end 117.602 98.298) (width 0.25) (layer F.Cu) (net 4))
 (segment (start 117.602 98.298) (end 118.872 99.568) (width 0.25) (layer F.Cu) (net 4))
 (segment (start 118.872 99.568) (end 118.872 112.014) (width 0.25) (layer F.Cu) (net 4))
 (segment (start 117.094 100.838) (end 121.158 100.838) (width 0.25) (layer B.Cu) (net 5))
 (segment (start 121.412 101.092) (end 121.412 112.014) (width 0.25) (layer F.Cu) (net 5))
 (segment (start 121.158 100.838) (end 121.412 101.092) (width 0.25) (layer F.Cu) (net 5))
 (via (at 121.158 100.838) (size 0.6) (drill 0.4) (layers F.Cu B.Cu) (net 5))
 (segment (start 117.094 103.378) (end 121.92 103.378) (width 0.25) (layer B.Cu) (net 7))
 (segment (start 123.444 104.902) (end 123.444 111.506) (width 0.25) (layer B.Cu) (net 7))
 (segment (start 121.92 103.378) (end 123.444 104.902) (width 0.25) (layer B.Cu) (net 7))
 (segment (start 123.444 111.506) (end 123.952 112.014) (width 0.25) (layer B.Cu) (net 7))
 (segment (start 114.554 105.918) (end 114.554 107.696) (width 0.25) (layer F.Cu) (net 8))
 (segment (start 139.192 114.808) (end 139.192 112.014) (width 0.25) (layer F.Cu) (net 8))
 (segment (start 137.922 116.078) (end 139.192 114.808) (width 0.25) (layer F.Cu) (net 8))
 (segment (start 116.078 116.078) (end 137.922 116.078) (width 0.25) (layer F.Cu) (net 8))
 (segment (start 115.062 115.062) (end 116.078 116.078) (width 0.25) (layer F.Cu) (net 8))
 (segment (start 115.062 108.204) (end 115.062 115.062) (width 0.25) (layer F.Cu) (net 8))
 (segment (start 114.554 107.696) (end 115.062 108.204) (width 0.25) (layer F.Cu) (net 8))
 (segment (start 117.094 105.918) (end 117.094 107.696) (width 0.25) (layer F.Cu) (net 9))
 (segment (start 126.492 113.538) (end 126.492 112.014) (width 0.25) (layer F.Cu) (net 9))
 (segment (start 125.476 114.554) (end 126.492 113.538) (width 0.25) (layer F.Cu) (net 9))
 (segment (start 118.618 114.554) (end 125.476 114.554) (width 0.25) (layer F.Cu) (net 9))
 (segment (start 117.602 113.538) (end 118.618 114.554) (width 0.25) (layer F.Cu) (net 9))
 (segment (start 117.602 108.204) (end 117.602 113.538) (width 0.25) (layer F.Cu) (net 9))
 (segment (start 117.094 107.696) (end 117.602 108.204) (width 0.25) (layer F.Cu) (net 9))
 (segment (start 142.24 105.41) (end 142.24 107.95) (width 0.25) (layer B.Cu) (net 9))
 (segment (start 126.492 116.078) (end 126.492 112.014) (width 0.25) (layer B.Cu) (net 9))
 (segment (start 127.508 117.094) (end 126.492 116.078) (width 0.25) (layer B.Cu) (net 9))
 (segment (start 141.986 117.094) (end 127.508 117.094) (width 0.25) (layer B.Cu) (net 9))
 (segment (start 143.002 116.078) (end 141.986 117.094) (width 0.25) (layer B.Cu) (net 9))
 (segment (start 143.002 108.712) (end 143.002 116.078) (width 0.25) (layer B.Cu) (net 9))
 (segment (start 142.24 107.95) (end 143.002 108.712) (width 0.25) (layer B.Cu) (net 9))
 (segment (start 113.792 112.014) (end 113.792 114.554) (width 0.25) (layer F.Cu) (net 10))
 (segment (start 117.348 128.778) (end 119.126 130.556) (width 0.25) (layer F.Cu) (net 10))
 (segment (start 117.348 126.492) (end 117.348 128.778) (width 0.25) (layer F.Cu) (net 10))
 (segment (start 111.506 120.65) (end 117.348 126.492) (width 0.25) (layer F.Cu) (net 10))
 (segment (start 111.506 116.84) (end 111.506 120.65) (width 0.25) (layer F.Cu) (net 10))
 (segment (start 113.792 114.554) (end 111.506 116.84) (width 0.25) (layer F.Cu) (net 10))
 (segment (start 113.792 112.014) (end 113.538 112.014) (width 0.25) (layer F.Cu) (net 10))
 (segment (start 113.792 119.634) (end 113.792 120.396) (width 0.25) (layer F.Cu) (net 11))
 (segment (start 113.792 120.396) (end 119.126 125.73) (width 0.25) (layer F.Cu) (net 11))
 (segment (start 119.126 125.73) (end 119.126 128.016) (width 0.25) (layer F.Cu) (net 11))
 (segment (start 116.332 119.634) (end 116.332 124.714) (width 0.25) (layer B.Cu) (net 12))
 (segment (start 121.666 132.334) (end 121.666 130.556) (width 0.25) (layer B.Cu) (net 12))
 (segment (start 120.904 133.096) (end 121.666 132.334) (width 0.25) (layer B.Cu) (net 12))
 (segment (start 118.364 133.096) (end 120.904 133.096) (width 0.25) (layer B.Cu) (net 12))
 (segment (start 117.348 132.08) (end 118.364 133.096) (width 0.25) (layer B.Cu) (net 12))
 (segment (start 117.348 125.73) (end 117.348 132.08) (width 0.25) (layer B.Cu) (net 12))
 (segment (start 116.332 124.714) (end 117.348 125.73) (width 0.25) (layer B.Cu) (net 12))
 (segment (start 118.872 119.634) (end 118.872 123.952) (width 0.25) (layer F.Cu) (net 13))
 (segment (start 121.666 126.746) (end 121.666 128.016) (width 0.25) (layer F.Cu) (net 13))
 (segment (start 118.872 123.952) (end 121.666 126.746) (width 0.25) (layer F.Cu) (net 13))
 (segment (start 121.412 119.634) (end 121.412 124.46) (width 0.25) (layer B.Cu) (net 14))
 (segment (start 122.936 129.286) (end 124.206 130.556) (width 0.25) (layer B.Cu) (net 14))
 (segment (start 122.936 125.984) (end 122.936 129.286) (width 0.25) (layer B.Cu) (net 14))
 (segment (start 121.412 124.46) (end 122.936 125.984) (width 0.25) (layer B.Cu) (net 14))
 (segment (start 123.952 119.634) (end 123.952 127.762) (width 0.25) (layer F.Cu) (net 15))
 (segment (start 123.952 127.762) (end 124.206 128.016) (width 0.25) (layer F.Cu) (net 15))
 (segment (start 126.492 119.634) (end 126.492 124.714) (width 0.25) (layer B.Cu) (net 16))
 (segment (start 125.476 129.286) (end 126.746 130.556) (width 0.25) (layer B.Cu) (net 16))
 (segment (start 125.476 125.73) (end 125.476 129.286) (width 0.25) (layer B.Cu) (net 16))
 (segment (start 126.492 124.714) (end 125.476 125.73) (width 0.25) (layer B.Cu) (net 16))
 (segment (start 129.032 119.634) (end 129.032 125.73) (width 0.25) (layer F.Cu) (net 17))
 (segment (start 129.032 125.73) (end 126.746 128.016) (width 0.25) (layer F.Cu) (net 17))
 (segment (start 131.572 119.634) (end 131.572 129.286) (width 0.25) (layer F.Cu) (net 18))
 (segment (start 133.096 130.81) (end 136.906 130.81) (width 0.25) (layer F.Cu) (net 18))
 (segment (start 131.572 129.286) (end 133.096 130.81) (width 0.25) (layer F.Cu) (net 18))
 (segment (start 134.112 119.634) (end 134.112 125.476) (width 0.25) (layer F.Cu) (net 19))
 (segment (start 134.112 125.476) (end 136.906 128.27) (width 0.25) (layer F.Cu) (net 19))
 (segment (start 136.652 119.634) (end 136.652 122.936) (width 0.25) (layer B.Cu) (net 20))
 (segment (start 139.446 132.842) (end 139.446 130.81) (width 0.25) (layer B.Cu) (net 20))
 (segment (start 138.43 133.858) (end 139.446 132.842) (width 0.25) (layer B.Cu) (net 20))
 (segment (start 135.382 133.858) (end 138.43 133.858) (width 0.25) (layer B.Cu) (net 20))
 (segment (start 133.35 131.826) (end 135.382 133.858) (width 0.25) (layer B.Cu) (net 20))
 (segment (start 133.35 126.238) (end 133.35 131.826) (width 0.25) (layer B.Cu) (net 20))
 (segment (start 136.652 122.936) (end 133.35 126.238) (width 0.25) (layer B.Cu) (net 20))
 (segment (start 139.192 119.634) (end 139.192 128.016) (width 0.25) (layer F.Cu) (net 21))
 (segment (start 139.192 128.016) (end 139.446 128.27) (width 0.25) (layer F.Cu) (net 21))
 (segment (start 141.732 119.634) (end 141.732 123.19) (width 0.25) (layer B.Cu) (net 22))
 (segment (start 140.716 129.54) (end 141.986 130.81) (width 0.25) (layer B.Cu) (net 22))
 (segment (start 140.716 124.206) (end 140.716 129.54) (width 0.25) (layer B.Cu) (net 22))
 (segment (start 141.732 123.19) (end 140.716 124.206) (width 0.25) (layer B.Cu) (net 22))
 (segment (start 144.272 119.634) (end 144.272 122.682) (width 0.25) (layer F.Cu) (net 23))
 (segment (start 141.986 124.968) (end 141.986 128.27) (width 0.25) (layer F.Cu) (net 23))
 (segment (start 144.272 122.682) (end 141.986 124.968) (width 0.25) (layer F.Cu) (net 23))
 (segment (start 146.812 119.634) (end 146.812 128.524) (width 0.25) (layer B.Cu) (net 24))
 (segment (start 146.812 128.524) (end 144.526 130.81) (width 0.25) (layer B.Cu) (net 24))
 (segment (start 146.812 112.014) (end 148.844 114.046) (width 0.25) (layer F.Cu) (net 25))
 (segment (start 148.844 123.952) (end 144.526 128.27) (width 0.25) (layer F.Cu) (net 25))
 (segment (start 148.844 114.046) (end 148.844 123.952) (width 0.25) (layer F.Cu) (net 25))
 (segment (start 131.572 99.314) (end 131.572 100.584) (width 0.25) (layer B.Cu) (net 26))
 (segment (start 134.112 109.728) (end 134.112 112.014) (width 0.25) (layer B.Cu) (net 26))
 (segment (start 132.334 107.95) (end 134.112 109.728) (width 0.25) (layer B.Cu) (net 26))
 (segment (start 132.334 101.346) (end 132.334 107.95) (width 0.25) (layer B.Cu) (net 26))
 (segment (start 131.572 100.584) (end 132.334 101.346) (width 0.25) (layer B.Cu) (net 26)))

